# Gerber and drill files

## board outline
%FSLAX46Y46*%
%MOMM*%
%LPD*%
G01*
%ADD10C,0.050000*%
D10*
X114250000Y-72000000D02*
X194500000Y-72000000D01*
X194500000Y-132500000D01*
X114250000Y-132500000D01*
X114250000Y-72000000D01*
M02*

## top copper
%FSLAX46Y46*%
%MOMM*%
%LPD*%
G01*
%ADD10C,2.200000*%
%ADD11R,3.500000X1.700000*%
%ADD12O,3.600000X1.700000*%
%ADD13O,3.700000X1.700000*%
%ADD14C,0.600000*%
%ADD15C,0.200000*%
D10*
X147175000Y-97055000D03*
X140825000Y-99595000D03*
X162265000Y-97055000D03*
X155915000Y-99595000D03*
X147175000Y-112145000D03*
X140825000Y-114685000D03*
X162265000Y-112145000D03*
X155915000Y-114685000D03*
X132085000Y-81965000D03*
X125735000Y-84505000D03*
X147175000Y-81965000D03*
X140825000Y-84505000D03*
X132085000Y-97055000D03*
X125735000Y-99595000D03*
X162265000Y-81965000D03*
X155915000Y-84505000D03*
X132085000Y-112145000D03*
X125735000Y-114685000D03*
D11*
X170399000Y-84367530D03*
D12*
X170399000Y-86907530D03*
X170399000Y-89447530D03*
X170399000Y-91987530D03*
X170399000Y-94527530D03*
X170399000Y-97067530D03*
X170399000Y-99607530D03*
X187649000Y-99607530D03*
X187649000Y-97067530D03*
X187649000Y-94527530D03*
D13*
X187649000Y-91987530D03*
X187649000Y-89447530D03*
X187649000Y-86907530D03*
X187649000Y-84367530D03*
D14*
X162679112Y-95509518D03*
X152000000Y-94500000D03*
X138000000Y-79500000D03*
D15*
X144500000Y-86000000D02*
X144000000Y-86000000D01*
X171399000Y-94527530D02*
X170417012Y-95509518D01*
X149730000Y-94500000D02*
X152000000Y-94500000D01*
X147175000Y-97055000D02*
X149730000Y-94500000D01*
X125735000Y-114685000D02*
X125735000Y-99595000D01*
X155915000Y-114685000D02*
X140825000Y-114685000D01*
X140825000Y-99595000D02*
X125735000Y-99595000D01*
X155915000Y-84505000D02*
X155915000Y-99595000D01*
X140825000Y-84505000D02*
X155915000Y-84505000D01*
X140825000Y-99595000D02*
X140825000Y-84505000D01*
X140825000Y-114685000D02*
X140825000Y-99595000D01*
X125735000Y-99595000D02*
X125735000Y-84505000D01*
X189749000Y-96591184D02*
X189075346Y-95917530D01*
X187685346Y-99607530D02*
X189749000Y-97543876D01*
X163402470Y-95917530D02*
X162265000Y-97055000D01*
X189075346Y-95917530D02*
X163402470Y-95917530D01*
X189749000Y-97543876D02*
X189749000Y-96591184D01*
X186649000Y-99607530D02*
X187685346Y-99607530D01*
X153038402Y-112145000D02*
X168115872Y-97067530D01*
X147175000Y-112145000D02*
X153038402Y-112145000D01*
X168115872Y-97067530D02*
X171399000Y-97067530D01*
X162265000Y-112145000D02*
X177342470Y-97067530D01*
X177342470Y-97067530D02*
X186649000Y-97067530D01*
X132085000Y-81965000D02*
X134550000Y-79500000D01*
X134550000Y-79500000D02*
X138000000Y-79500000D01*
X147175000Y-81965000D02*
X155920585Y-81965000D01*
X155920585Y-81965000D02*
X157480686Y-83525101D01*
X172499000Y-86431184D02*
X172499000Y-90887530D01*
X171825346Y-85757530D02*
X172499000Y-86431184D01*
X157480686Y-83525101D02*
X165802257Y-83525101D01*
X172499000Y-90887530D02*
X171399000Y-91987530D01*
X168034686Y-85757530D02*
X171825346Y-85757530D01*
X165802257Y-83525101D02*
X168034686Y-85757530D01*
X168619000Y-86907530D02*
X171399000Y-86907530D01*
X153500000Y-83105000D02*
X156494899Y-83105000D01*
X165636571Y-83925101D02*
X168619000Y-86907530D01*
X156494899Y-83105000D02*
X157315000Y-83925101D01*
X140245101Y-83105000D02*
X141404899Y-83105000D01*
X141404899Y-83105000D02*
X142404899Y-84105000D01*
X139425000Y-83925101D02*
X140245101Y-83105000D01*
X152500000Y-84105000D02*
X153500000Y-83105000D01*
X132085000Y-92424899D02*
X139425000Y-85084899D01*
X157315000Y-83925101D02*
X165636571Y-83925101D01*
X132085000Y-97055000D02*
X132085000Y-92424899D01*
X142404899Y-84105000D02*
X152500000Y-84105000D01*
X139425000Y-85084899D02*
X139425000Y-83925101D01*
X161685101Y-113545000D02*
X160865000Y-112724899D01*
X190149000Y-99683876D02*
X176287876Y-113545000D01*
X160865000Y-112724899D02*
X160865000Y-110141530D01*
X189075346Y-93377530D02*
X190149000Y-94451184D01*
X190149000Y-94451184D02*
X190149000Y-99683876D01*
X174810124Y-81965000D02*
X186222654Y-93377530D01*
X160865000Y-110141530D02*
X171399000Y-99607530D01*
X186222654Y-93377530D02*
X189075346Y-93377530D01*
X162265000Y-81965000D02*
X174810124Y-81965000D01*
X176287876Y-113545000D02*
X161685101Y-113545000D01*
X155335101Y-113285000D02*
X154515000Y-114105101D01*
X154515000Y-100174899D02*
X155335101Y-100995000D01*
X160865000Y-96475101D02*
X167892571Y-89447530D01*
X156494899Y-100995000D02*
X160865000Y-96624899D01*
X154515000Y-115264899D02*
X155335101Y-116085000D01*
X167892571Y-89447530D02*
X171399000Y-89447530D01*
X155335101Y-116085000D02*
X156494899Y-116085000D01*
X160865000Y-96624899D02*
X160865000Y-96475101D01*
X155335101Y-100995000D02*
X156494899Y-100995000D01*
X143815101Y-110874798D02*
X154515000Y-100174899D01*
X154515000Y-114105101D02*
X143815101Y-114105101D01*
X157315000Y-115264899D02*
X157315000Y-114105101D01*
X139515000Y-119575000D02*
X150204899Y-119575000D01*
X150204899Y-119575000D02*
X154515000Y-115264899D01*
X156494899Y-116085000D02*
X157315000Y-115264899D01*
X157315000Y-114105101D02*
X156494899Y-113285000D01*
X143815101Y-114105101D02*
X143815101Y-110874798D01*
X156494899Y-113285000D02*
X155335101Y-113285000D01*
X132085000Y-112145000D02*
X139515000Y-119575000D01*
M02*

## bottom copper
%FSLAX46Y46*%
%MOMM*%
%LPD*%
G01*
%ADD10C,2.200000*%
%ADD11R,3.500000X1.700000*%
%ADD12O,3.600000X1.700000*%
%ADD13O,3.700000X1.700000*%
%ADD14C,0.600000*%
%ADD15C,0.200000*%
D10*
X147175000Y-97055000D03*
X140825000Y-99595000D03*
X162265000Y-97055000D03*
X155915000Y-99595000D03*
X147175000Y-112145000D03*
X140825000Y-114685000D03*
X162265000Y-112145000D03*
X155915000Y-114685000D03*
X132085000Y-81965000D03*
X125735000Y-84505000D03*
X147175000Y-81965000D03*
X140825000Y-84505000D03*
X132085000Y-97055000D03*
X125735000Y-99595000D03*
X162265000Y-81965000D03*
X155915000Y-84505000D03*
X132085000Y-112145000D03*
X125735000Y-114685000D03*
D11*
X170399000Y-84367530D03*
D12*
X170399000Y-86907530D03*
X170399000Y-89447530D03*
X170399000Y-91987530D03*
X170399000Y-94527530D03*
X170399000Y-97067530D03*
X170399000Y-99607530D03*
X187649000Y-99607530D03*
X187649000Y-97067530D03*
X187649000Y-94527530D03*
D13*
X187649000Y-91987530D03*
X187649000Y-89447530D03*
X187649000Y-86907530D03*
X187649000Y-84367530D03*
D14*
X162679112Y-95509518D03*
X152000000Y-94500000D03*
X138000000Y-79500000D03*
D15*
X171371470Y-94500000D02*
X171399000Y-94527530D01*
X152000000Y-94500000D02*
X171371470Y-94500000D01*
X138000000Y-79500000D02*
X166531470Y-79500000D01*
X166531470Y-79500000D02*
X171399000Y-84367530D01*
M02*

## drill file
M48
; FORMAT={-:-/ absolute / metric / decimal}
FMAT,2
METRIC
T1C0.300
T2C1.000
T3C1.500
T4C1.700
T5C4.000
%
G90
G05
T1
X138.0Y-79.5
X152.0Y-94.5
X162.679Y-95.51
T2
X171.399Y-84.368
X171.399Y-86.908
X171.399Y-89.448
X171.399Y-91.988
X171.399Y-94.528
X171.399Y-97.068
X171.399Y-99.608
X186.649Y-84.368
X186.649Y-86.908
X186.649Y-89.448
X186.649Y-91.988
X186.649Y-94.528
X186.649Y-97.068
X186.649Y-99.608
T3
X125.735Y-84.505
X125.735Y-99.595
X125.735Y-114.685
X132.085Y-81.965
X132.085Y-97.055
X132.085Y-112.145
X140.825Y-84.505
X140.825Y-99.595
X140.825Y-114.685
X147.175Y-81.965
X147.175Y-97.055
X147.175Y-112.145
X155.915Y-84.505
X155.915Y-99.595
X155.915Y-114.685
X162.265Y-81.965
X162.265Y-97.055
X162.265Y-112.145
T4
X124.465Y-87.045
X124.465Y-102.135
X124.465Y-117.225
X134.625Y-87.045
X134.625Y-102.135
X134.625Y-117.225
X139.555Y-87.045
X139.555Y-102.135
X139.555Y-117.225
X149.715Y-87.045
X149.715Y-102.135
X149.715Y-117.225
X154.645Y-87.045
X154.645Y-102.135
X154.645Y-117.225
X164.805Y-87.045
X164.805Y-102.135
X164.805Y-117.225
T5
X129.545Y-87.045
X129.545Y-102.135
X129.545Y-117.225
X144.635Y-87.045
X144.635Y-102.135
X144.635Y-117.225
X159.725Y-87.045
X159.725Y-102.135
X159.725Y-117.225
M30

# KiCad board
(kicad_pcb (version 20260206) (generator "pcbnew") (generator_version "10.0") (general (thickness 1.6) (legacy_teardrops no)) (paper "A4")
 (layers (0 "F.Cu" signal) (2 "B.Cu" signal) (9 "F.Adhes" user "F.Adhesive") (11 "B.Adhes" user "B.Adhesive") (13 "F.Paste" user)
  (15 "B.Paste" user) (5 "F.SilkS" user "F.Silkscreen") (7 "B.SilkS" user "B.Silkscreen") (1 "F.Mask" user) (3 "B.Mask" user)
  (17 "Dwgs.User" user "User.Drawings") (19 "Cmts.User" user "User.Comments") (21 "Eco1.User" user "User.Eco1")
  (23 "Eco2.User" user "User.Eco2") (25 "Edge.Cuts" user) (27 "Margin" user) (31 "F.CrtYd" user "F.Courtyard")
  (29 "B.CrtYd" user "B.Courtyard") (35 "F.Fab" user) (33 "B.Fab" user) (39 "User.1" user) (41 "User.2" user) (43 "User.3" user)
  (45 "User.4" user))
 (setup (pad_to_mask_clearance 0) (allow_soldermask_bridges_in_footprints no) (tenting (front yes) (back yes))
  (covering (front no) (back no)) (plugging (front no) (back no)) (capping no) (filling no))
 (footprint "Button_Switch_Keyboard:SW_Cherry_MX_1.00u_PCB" (layer "F.Cu") (at 147.175 97.055)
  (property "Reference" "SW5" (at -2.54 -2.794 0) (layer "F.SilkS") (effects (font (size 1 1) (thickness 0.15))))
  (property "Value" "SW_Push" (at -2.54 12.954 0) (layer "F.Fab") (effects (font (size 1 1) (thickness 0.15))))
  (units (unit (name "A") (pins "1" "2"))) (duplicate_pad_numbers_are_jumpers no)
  (pad "" np_thru_hole circle (at -7.62 5.08) (size 1.7 1.7) (drill 1.7) (layers "*.Cu" "*.Mask"))
  (pad "" np_thru_hole circle (at -2.54 5.08) (size 4 4) (drill 4) (layers "*.Cu" "*.Mask"))
  (pad "" np_thru_hole circle (at 2.54 5.08) (size 1.7 1.7) (drill 1.7) (layers "*.Cu" "*.Mask"))
  (pad "1" thru_hole circle (at 0 0) (size 2.2 2.2) (drill 1.5) (layers "*.Cu" "*.Mask") (remove_unused_layers no)
   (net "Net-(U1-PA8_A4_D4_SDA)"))
  (pad "2" thru_hole circle (at -6.35 2.54) (size 2.2 2.2) (drill 1.5) (layers "*.Cu" "*.Mask") (remove_unused_layers no)
   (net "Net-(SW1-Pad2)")))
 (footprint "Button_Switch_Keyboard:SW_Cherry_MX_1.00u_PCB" (layer "F.Cu") (at 162.265 97.055)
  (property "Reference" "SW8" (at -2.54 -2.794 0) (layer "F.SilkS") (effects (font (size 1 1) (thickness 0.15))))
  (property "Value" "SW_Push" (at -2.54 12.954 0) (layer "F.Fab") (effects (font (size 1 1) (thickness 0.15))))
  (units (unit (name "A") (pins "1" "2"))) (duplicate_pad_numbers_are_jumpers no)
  (pad "" np_thru_hole circle (at -7.62 5.08) (size 1.7 1.7) (drill 1.7) (layers "*.Cu" "*.Mask"))
  (pad "" np_thru_hole circle (at -2.54 5.08) (size 4 4) (drill 4) (layers "*.Cu" "*.Mask"))
  (pad "" np_thru_hole circle (at 2.54 5.08) (size 1.7 1.7) (drill 1.7) (layers "*.Cu" "*.Mask"))
  (pad "1" thru_hole circle (at 0 0) (size 2.2 2.2) (drill 1.5) (layers "*.Cu" "*.Mask") (remove_unused_layers no)
   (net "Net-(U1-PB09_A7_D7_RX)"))
  (pad "2" thru_hole circle (at -6.35 2.54) (size 2.2 2.2) (drill 1.5) (layers "*.Cu" "*.Mask") (remove_unused_layers no)
   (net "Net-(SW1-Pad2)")))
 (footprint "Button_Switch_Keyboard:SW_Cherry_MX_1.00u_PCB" (layer "F.Cu") (at 147.175 112.145)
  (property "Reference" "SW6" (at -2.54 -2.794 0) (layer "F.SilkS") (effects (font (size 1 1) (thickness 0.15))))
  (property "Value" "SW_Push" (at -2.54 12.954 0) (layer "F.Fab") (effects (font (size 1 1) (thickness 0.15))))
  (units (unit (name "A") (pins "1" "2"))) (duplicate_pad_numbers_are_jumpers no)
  (pad "" np_thru_hole circle (at -7.62 5.08) (size 1.7 1.7) (drill 1.7) (layers "*.Cu" "*.Mask"))
  (pad "" np_thru_hole circle (at -2.54 5.08) (size 4 4) (drill 4) (layers "*.Cu" "*.Mask"))
  (pad "" np_thru_hole circle (at 2.54 5.08) (size 1.7 1.7) (drill 1.7) (layers "*.Cu" "*.Mask"))
  (pad "1" thru_hole circle (at 0 0) (size 2.2 2.2) (drill 1.5) (layers "*.Cu" "*.Mask") (remove_unused_layers no)
   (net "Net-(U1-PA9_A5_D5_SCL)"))
  (pad "2" thru_hole circle (at -6.35 2.54) (size 2.2 2.2) (drill 1.5) (layers "*.Cu" "*.Mask") (remove_unused_layers no)
   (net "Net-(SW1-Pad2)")))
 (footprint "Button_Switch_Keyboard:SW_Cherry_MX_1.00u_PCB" (layer "F.Cu") (at 162.265 112.145)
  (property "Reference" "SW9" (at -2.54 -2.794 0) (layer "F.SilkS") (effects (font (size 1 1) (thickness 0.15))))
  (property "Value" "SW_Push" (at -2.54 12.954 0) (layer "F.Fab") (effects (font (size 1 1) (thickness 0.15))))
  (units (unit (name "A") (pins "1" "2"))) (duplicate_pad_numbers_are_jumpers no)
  (pad "" np_thru_hole circle (at -7.62 5.08) (size 1.7 1.7) (drill 1.7) (layers "*.Cu" "*.Mask"))
  (pad "" np_thru_hole circle (at -2.54 5.08) (size 4 4) (drill 4) (layers "*.Cu" "*.Mask"))
  (pad "" np_thru_hole circle (at 2.54 5.08) (size 1.7 1.7) (drill 1.7) (layers "*.Cu" "*.Mask"))
  (pad "1" thru_hole circle (at 0 0) (size 2.2 2.2) (drill 1.5) (layers "*.Cu" "*.Mask") (remove_unused_layers no)
   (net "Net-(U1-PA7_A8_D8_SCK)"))
  (pad "2" thru_hole circle (at -6.35 2.54) (size 2.2 2.2) (drill 1.5) (layers "*.Cu" "*.Mask") (remove_unused_layers no)
   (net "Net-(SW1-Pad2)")))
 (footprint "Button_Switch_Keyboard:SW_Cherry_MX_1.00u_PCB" (layer "F.Cu") (at 132.085 81.965)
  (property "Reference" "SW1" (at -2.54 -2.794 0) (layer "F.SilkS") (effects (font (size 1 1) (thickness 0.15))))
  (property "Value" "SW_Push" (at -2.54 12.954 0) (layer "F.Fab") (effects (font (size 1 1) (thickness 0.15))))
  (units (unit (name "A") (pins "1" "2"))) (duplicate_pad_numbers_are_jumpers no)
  (pad "" np_thru_hole circle (at -7.62 5.08) (size 1.7 1.7) (drill 1.7) (layers "*.Cu" "*.Mask"))
  (pad "" np_thru_hole circle (at -2.54 5.08) (size 4 4) (drill 4) (layers "*.Cu" "*.Mask"))
  (pad "" np_thru_hole circle (at 2.54 5.08) (size 1.7 1.7) (drill 1.7) (layers "*.Cu" "*.Mask"))
  (pad "1" thru_hole circle (at 0 0) (size 2.2 2.2) (drill 1.5) (layers "*.Cu" "*.Mask") (remove_unused_layers no)
   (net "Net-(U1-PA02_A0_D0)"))
  (pad "2" thru_hole circle (at -6.35 2.54) (size 2.2 2.2) (drill 1.5) (layers "*.Cu" "*.Mask") (remove_unused_layers no)
   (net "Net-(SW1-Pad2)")))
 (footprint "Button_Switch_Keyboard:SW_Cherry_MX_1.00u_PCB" (layer "F.Cu") (at 147.175 81.965)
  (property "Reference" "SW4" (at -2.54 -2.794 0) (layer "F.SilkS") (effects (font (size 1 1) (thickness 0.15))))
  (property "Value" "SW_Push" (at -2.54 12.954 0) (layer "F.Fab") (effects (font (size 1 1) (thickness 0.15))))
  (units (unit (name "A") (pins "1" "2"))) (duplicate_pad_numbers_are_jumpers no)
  (pad "" np_thru_hole circle (at -7.62 5.08) (size 1.7 1.7) (drill 1.7) (layers "*.Cu" "*.Mask"))
  (pad "" np_thru_hole circle (at -2.54 5.08) (size 4 4) (drill 4) (layers "*.Cu" "*.Mask"))
  (pad "" np_thru_hole circle (at 2.54 5.08) (size 1.7 1.7) (drill 1.7) (layers "*.Cu" "*.Mask"))
  (pad "1" thru_hole circle (at 0 0) (size 2.2 2.2) (drill 1.5) (layers "*.Cu" "*.Mask") (remove_unused_layers no)
   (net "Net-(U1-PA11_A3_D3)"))
  (pad "2" thru_hole circle (at -6.35 2.54) (size 2.2 2.2) (drill 1.5) (layers "*.Cu" "*.Mask") (remove_unused_layers no)
   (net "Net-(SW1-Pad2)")))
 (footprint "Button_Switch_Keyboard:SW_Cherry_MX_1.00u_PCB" (layer "F.Cu") (at 132.085 97.055)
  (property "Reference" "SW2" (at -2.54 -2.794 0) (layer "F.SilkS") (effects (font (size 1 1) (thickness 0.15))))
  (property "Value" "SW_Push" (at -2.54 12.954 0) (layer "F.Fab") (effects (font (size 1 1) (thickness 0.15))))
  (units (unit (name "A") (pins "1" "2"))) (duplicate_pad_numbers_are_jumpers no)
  (pad "" np_thru_hole circle (at -7.62 5.08) (size 1.7 1.7) (drill 1.7) (layers "*.Cu" "*.Mask"))
  (pad "" np_thru_hole circle (at -2.54 5.08) (size 4 4) (drill 4) (layers "*.Cu" "*.Mask"))
  (pad "" np_thru_hole circle (at 2.54 5.08) (size 1.7 1.7) (drill 1.7) (layers "*.Cu" "*.Mask"))
  (pad "1" thru_hole circle (at 0 0) (size 2.2 2.2) (drill 1.5) (layers "*.Cu" "*.Mask") (remove_unused_layers no)
   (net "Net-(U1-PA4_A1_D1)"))
  (pad "2" thru_hole circle (at -6.35 2.54) (size 2.2 2.2) (drill 1.5) (layers "*.Cu" "*.Mask") (remove_unused_layers no)
   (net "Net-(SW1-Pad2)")))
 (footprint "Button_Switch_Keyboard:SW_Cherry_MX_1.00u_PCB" (layer "F.Cu") (at 162.265 81.965)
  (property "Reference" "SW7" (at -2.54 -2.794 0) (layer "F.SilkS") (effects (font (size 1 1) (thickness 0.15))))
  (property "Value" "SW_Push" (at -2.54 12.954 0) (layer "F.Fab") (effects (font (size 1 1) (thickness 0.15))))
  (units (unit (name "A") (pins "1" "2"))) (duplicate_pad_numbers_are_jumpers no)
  (pad "" np_thru_hole circle (at -7.62 5.08) (size 1.7 1.7) (drill 1.7) (layers "*.Cu" "*.Mask"))
  (pad "" np_thru_hole circle (at -2.54 5.08) (size 4 4) (drill 4) (layers "*.Cu" "*.Mask"))
  (pad "" np_thru_hole circle (at 2.54 5.08) (size 1.7 1.7) (drill 1.7) (layers "*.Cu" "*.Mask"))
  (pad "1" thru_hole circle (at 0 0) (size 2.2 2.2) (drill 1.5) (layers "*.Cu" "*.Mask") (remove_unused_layers no)
   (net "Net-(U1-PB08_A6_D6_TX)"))
  (pad "2" thru_hole circle (at -6.35 2.54) (size 2.2 2.2) (drill 1.5) (layers "*.Cu" "*.Mask") (remove_unused_layers no)
   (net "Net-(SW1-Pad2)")))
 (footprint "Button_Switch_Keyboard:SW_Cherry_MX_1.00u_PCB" (layer "F.Cu") (at 132.085 112.145)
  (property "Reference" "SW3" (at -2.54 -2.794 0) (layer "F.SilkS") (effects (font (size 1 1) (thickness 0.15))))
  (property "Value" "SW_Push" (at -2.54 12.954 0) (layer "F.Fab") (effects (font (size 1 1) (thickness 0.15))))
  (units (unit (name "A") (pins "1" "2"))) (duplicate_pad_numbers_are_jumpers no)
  (pad "" np_thru_hole circle (at -7.62 5.08) (size 1.7 1.7) (drill 1.7) (layers "*.Cu" "*.Mask"))
  (pad "" np_thru_hole circle (at -2.54 5.08) (size 4 4) (drill 4) (layers "*.Cu" "*.Mask"))
  (pad "" np_thru_hole circle (at 2.54 5.08) (size 1.7 1.7) (drill 1.7) (layers "*.Cu" "*.Mask"))
  (pad "1" thru_hole circle (at 0 0) (size 2.2 2.2) (drill 1.5) (layers "*.Cu" "*.Mask") (remove_unused_layers no)
   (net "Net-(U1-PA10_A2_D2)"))
  (pad "2" thru_hole circle (at -6.35 2.54) (size 2.2 2.2) (drill 1.5) (layers "*.Cu" "*.Mask") (remove_unused_layers no)
   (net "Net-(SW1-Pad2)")))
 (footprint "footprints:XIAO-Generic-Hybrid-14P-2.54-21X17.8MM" (layer "F.Cu") (at 179.024 91.98753)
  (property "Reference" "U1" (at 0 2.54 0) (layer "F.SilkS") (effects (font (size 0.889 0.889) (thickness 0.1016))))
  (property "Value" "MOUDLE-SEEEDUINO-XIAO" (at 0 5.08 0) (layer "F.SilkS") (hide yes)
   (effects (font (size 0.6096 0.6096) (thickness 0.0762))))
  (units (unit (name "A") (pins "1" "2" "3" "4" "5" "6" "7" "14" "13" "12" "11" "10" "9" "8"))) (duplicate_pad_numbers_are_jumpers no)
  (pad "1" thru_hole rect (at -7.625 -7.62) (size 3.5 1.7) (drill 1 (offset -1 0)) (layers "*.Cu" "*.Mask") (remove_unused_layers no)
   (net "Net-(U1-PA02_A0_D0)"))
  (pad "2" thru_hole oval (at -7.625 -5.08) (size 3.6 1.7) (drill 1 (offset -1 0)) (layers "*.Cu" "*.Mask") (remove_unused_layers no)
   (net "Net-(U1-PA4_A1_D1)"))
  (pad "3" thru_hole oval (at -7.625 -2.54) (size 3.6 1.7) (drill 1 (offset -1 0)) (layers "*.Cu" "*.Mask") (remove_unused_layers no)
   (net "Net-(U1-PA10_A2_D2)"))
  (pad "4" thru_hole oval (at -7.625 0) (size 3.6 1.7) (drill 1 (offset -1 0)) (layers "*.Cu" "*.Mask") (remove_unused_layers no)
   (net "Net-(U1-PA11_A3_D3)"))
  (pad "5" thru_hole oval (at -7.625 2.54) (size 3.6 1.7) (drill 1 (offset -1 0)) (layers "*.Cu" "*.Mask") (remove_unused_layers no)
   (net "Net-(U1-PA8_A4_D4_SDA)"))
  (pad "6" thru_hole oval (at -7.625 5.08 180) (size 3.6 1.7) (drill 1 (offset 1 0)) (layers "*.Cu" "*.Mask") (remove_unused_layers no)
   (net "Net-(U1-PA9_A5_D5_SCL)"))
  (pad "7" thru_hole oval (at -7.625 7.62) (size 3.6 1.7) (drill 1 (offset -1 0)) (layers "*.Cu" "*.Mask") (remove_unused_layers no)
   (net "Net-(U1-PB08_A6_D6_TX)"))
  (pad "8" thru_hole oval (at 7.625 7.62) (size 3.6 1.7) (drill 1 (offset 1 0)) (layers "*.Cu" "*.Mask") (remove_unused_layers no)
   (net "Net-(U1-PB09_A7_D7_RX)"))
  (pad "9" thru_hole oval (at 7.625 5.08) (size 3.6 1.7) (drill 1 (offset 1 0)) (layers "*.Cu" "*.Mask") (remove_unused_layers no)
   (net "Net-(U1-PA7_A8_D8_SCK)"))
  (pad "10" thru_hole oval (at 7.625 2.54) (size 3.6 1.7) (drill 1 (offset 1 0)) (layers "*.Cu" "*.Mask") (remove_unused_layers no)
   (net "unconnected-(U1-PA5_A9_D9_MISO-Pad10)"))
  (pad "11" thru_hole oval (at 7.625 0) (size 3.7 1.7) (drill 1 (offset 1 0)) (layers "*.Cu" "*.Mask") (remove_unused_layers no)
   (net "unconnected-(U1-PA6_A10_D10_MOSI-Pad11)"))
  (pad "12" thru_hole oval (at 7.625 -2.54) (size 3.7 1.7) (drill 1 (offset 1 0)) (layers "*.Cu" "*.Mask") (remove_unused_layers no)
   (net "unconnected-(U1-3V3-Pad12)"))
  (pad "13" thru_hole oval (at 7.625 -5.08) (size 3.7 1.7) (drill 1 (offset 1 0)) (layers "*.Cu" "*.Mask") (remove_unused_layers no)
   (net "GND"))
  (pad "14" thru_hole oval (at 7.625 -7.62) (size 3.7 1.7) (drill 1 (offset 1 0)) (layers "*.Cu" "*.Mask") (remove_unused_layers no)
   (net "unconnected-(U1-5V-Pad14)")))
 (gr_rect (start 114.25 72) (end 194.5 132.5) (stroke (width 0.05) (type default)) (fill no) (layer "Edge.Cuts"))
 (segment (start 144.5 86) (end 144 86) (width 0.2) (layer "F.Cu") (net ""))
 (segment (start 171.399 94.52753) (end 170.417012 95.509518) (width 0.2) (layer "F.Cu") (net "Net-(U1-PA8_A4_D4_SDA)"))
 (segment (start 149.73 94.5) (end 152 94.5) (width 0.2) (layer "F.Cu") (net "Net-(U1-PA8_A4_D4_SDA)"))
 (segment (start 147.175 97.055) (end 149.73 94.5) (width 0.2) (layer "F.Cu") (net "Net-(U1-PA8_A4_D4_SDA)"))
 (via (at 162.679112 95.509518) (size 0.6) (drill 0.3) (layers "F.Cu" "B.Cu") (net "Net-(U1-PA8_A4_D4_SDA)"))
 (via (at 152 94.5) (size 0.6) (drill 0.3) (layers "F.Cu" "B.Cu") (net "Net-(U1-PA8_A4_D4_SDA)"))
 (segment (start 171.37147 94.5) (end 171.399 94.52753) (width 0.2) (layer "B.Cu") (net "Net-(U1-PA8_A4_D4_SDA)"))
 (segment (start 152 94.5) (end 171.37147 94.5) (width 0.2) (layer "B.Cu") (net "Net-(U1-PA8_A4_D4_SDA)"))
 (segment (start 125.735 114.685) (end 125.735 99.595) (width 0.2) (layer "F.Cu") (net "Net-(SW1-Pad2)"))
 (segment (start 155.915 114.685) (end 140.825 114.685) (width 0.2) (layer "F.Cu") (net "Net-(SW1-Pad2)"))
 (segment (start 140.825 99.595) (end 125.735 99.595) (width 0.2) (layer "F.Cu") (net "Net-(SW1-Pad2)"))
 (segment (start 155.915 84.505) (end 155.915 99.595) (width 0.2) (layer "F.Cu") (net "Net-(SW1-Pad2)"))
 (segment (start 140.825 84.505) (end 155.915 84.505) (width 0.2) (layer "F.Cu") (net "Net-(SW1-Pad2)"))
 (segment (start 140.825 99.595) (end 140.825 84.505) (width 0.2) (layer "F.Cu") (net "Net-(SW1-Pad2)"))
 (segment (start 140.825 114.685) (end 140.825 99.595) (width 0.2) (layer "F.Cu") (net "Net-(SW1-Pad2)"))
 (segment (start 125.735 99.595) (end 125.735 84.505) (width 0.2) (layer "F.Cu") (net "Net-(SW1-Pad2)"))
 (segment (start 189.749 96.591184) (end 189.075346 95.91753) (width 0.2) (layer "F.Cu") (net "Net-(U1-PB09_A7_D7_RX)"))
 (segment (start 187.685346 99.60753) (end 189.749 97.543876) (width 0.2) (layer "F.Cu") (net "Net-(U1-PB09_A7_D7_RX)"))
 (segment (start 163.40247 95.91753) (end 162.265 97.055) (width 0.2) (layer "F.Cu") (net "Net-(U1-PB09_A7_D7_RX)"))
 (segment (start 189.075346 95.91753) (end 163.40247 95.91753) (width 0.2) (layer "F.Cu") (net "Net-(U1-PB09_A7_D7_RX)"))
 (segment (start 189.749 97.543876) (end 189.749 96.591184) (width 0.2) (layer "F.Cu") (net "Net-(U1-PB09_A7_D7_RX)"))
 (segment (start 186.649 99.60753) (end 187.685346 99.60753) (width 0.2) (layer "F.Cu") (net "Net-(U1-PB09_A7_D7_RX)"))
 (segment (start 153.038402 112.145) (end 168.115872 97.06753) (width 0.2) (layer "F.Cu") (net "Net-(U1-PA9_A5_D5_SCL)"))
 (segment (start 147.175 112.145) (end 153.038402 112.145) (width 0.2) (layer "F.Cu") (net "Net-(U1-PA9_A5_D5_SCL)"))
 (segment (start 168.115872 97.06753) (end 171.399 97.06753) (width 0.2) (layer "F.Cu") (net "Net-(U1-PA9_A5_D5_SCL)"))
 (segment (start 162.265 112.145) (end 177.34247 97.06753) (width 0.2) (layer "F.Cu") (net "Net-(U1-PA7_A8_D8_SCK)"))
 (segment (start 177.34247 97.06753) (end 186.649 97.06753) (width 0.2) (layer "F.Cu") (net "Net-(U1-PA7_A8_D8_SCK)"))
 (segment (start 132.085 81.965) (end 134.55 79.5) (width 0.2) (layer "F.Cu") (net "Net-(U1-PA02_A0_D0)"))
 (segment (start 134.55 79.5) (end 138 79.5) (width 0.2) (layer "F.Cu") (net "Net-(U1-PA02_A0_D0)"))
 (via (at 138 79.5) (size 0.6) (drill 0.3) (layers "F.Cu" "B.Cu") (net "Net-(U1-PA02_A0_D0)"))
 (segment (start 138 79.5) (end 166.53147 79.5) (width 0.2) (layer "B.Cu") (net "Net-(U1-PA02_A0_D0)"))
 (segment (start 166.53147 79.5) (end 171.399 84.36753) (width 0.2) (layer "B.Cu") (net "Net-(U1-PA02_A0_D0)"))
 (segment (start 147.175 81.965) (end 155.920585 81.965) (width 0.2) (layer "F.Cu") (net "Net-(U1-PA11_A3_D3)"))
 (segment (start 155.920585 81.965) (end 157.480686 83.525101) (width 0.2) (layer "F.Cu") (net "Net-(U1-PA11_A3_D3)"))
 (segment (start 172.499 86.431184) (end 172.499 90.88753) (width 0.2) (layer "F.Cu") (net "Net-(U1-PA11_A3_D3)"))
 (segment (start 171.825346 85.75753) (end 172.499 86.431184) (width 0.2) (layer "F.Cu") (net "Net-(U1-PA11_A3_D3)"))
 (segment (start 157.480686 83.525101) (end 165.802257 83.525101) (width 0.2) (layer "F.Cu") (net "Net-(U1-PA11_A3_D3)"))
 (segment (start 172.499 90.88753) (end 171.399 91.98753) (width 0.2) (layer "F.Cu") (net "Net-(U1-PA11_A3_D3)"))
 (segment (start 168.034686 85.75753) (end 171.825346 85.75753) (width 0.2) (layer "F.Cu") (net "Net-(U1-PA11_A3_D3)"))
 (segment (start 165.802257 83.525101) (end 168.034686 85.75753) (width 0.2) (layer "F.Cu") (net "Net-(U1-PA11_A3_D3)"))
 (segment (start 168.619 86.90753) (end 171.399 86.90753) (width 0.2) (layer "F.Cu") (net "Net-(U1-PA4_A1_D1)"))
 (segment (start 153.5 83.105) (end 156.494899 83.105) (width 0.2) (layer "F.Cu") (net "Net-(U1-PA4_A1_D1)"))
 (segment (start 165.636571 83.925101) (end 168.619 86.90753) (width 0.2) (layer "F.Cu") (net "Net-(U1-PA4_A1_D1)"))
 (segment (start 156.494899 83.105) (end 157.315 83.925101) (width 0.2) (layer "F.Cu") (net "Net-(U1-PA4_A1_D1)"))
 (segment (start 140.245101 83.105) (end 141.404899 83.105) (width 0.2) (layer "F.Cu") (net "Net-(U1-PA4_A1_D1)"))
 (segment (start 141.404899 83.105) (end 142.404899 84.105) (width 0.2) (layer "F.Cu") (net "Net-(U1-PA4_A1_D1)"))
 (segment (start 139.425 83.925101) (end 140.245101 83.105) (width 0.2) (layer "F.Cu") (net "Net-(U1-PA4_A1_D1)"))
 (segment (start 152.5 84.105) (end 153.5 83.105) (width 0.2) (layer "F.Cu") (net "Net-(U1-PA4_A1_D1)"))
 (segment (start 132.085 92.424899) (end 139.425 85.084899) (width 0.2) (layer "F.Cu") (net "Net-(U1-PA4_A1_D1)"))
 (segment (start 157.315 83.925101) (end 165.636571 83.925101) (width 0.2) (layer "F.Cu") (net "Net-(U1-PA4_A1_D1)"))
 (segment (start 132.085 97.055) (end 132.085 92.424899) (width 0.2) (layer "F.Cu") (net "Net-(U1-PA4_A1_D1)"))
 (segment (start 142.404899 84.105) (end 152.5 84.105) (width 0.2) (layer "F.Cu") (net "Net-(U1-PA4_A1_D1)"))
 (segment (start 139.425 85.084899) (end 139.425 83.925101) (width 0.2) (layer "F.Cu") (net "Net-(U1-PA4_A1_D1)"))
 (segment (start 161.685101 113.545) (end 160.865 112.724899) (width 0.2) (layer "F.Cu") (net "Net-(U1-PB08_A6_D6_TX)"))
 (segment (start 190.149 99.683876) (end 176.287876 113.545) (width 0.2) (layer "F.Cu") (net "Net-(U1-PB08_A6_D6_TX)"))
 (segment (start 160.865 112.724899) (end 160.865 110.14153) (width 0.2) (layer "F.Cu") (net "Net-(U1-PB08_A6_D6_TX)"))
 (segment (start 189.075346 93.37753) (end 190.149 94.451184) (width 0.2) (layer "F.Cu") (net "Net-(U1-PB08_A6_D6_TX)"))
 (segment (start 190.149 94.451184) (end 190.149 99.683876) (width 0.2) (layer "F.Cu") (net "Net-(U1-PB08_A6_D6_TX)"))
 (segment (start 174.810124 81.965) (end 186.222654 93.37753) (width 0.2) (layer "F.Cu") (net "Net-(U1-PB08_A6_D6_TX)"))
 (segment (start 160.865 110.14153) (end 171.399 99.60753) (width 0.2) (layer "F.Cu") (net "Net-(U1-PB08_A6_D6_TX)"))
 (segment (start 186.222654 93.37753) (end 189.075346 93.37753) (width 0.2) (layer "F.Cu") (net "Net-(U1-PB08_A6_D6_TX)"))
 (segment (start 162.265 81.965) (end 174.810124 81.965) (width 0.2) (layer "F.Cu") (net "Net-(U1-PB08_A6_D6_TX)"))
 (segment (start 176.287876 113.545) (end 161.685101 113.545) (width 0.2) (layer "F.Cu") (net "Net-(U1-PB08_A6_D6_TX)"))
 (segment (start 155.335101 113.285) (end 154.515 114.105101) (width 0.2) (layer "F.Cu") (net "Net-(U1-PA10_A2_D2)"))
 (segment (start 154.515 100.174899) (end 155.335101 100.995) (width 0.2) (layer "F.Cu") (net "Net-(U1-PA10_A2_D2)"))
 (segment (start 160.865 96.475101) (end 167.892571 89.44753) (width 0.2) (layer "F.Cu") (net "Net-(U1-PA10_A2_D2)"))
 (segment (start 156.494899 100.995) (end 160.865 96.624899) (width 0.2) (layer "F.Cu") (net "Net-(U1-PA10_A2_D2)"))
 (segment (start 154.515 115.264899) (end 155.335101 116.085) (width 0.2) (layer "F.Cu") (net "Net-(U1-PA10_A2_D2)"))
 (segment (start 167.892571 89.44753) (end 171.399 89.44753) (width 0.2) (layer "F.Cu") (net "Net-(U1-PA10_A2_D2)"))
 (segment (start 155.335101 116.085) (end 156.494899 116.085) (width 0.2) (layer "F.Cu") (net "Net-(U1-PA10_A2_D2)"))
 (segment (start 160.865 96.624899) (end 160.865 96.475101) (width 0.2) (layer "F.Cu") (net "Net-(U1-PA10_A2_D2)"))
 (segment (start 155.335101 100.995) (end 156.494899 100.995) (width 0.2) (layer "F.Cu") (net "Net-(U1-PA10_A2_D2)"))
 (segment (start 143.815101 110.874798) (end 154.515 100.174899) (width 0.2) (layer "F.Cu") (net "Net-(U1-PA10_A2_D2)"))
 (segment (start 154.515 114.105101) (end 143.815101 114.105101) (width 0.2) (layer "F.Cu") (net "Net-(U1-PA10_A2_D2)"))
 (segment (start 157.315 115.264899) (end 157.315 114.105101) (width 0.2) (layer "F.Cu") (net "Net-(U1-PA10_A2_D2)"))
 (segment (start 139.515 119.575) (end 150.204899 119.575) (width 0.2) (layer "F.Cu") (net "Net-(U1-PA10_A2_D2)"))
 (segment (start 150.204899 119.575) (end 154.515 115.264899) (width 0.2) (layer "F.Cu") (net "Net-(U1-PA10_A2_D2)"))
 (segment (start 156.494899 116.085) (end 157.315 115.264899) (width 0.2) (layer "F.Cu") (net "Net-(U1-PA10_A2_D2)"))
 (segment (start 157.315 114.105101) (end 156.494899 113.285) (width 0.2) (layer "F.Cu") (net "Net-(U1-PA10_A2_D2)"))
 (segment (start 143.815101 114.105101) (end 143.815101 110.874798) (width 0.2) (layer "F.Cu") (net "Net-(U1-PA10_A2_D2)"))
 (segment (start 156.494899 113.285) (end 155.335101 113.285) (width 0.2) (layer "F.Cu") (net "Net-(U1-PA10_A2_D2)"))
 (segment (start 132.085 112.145) (end 139.515 119.575) (width 0.2) (layer "F.Cu") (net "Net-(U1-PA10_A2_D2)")))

